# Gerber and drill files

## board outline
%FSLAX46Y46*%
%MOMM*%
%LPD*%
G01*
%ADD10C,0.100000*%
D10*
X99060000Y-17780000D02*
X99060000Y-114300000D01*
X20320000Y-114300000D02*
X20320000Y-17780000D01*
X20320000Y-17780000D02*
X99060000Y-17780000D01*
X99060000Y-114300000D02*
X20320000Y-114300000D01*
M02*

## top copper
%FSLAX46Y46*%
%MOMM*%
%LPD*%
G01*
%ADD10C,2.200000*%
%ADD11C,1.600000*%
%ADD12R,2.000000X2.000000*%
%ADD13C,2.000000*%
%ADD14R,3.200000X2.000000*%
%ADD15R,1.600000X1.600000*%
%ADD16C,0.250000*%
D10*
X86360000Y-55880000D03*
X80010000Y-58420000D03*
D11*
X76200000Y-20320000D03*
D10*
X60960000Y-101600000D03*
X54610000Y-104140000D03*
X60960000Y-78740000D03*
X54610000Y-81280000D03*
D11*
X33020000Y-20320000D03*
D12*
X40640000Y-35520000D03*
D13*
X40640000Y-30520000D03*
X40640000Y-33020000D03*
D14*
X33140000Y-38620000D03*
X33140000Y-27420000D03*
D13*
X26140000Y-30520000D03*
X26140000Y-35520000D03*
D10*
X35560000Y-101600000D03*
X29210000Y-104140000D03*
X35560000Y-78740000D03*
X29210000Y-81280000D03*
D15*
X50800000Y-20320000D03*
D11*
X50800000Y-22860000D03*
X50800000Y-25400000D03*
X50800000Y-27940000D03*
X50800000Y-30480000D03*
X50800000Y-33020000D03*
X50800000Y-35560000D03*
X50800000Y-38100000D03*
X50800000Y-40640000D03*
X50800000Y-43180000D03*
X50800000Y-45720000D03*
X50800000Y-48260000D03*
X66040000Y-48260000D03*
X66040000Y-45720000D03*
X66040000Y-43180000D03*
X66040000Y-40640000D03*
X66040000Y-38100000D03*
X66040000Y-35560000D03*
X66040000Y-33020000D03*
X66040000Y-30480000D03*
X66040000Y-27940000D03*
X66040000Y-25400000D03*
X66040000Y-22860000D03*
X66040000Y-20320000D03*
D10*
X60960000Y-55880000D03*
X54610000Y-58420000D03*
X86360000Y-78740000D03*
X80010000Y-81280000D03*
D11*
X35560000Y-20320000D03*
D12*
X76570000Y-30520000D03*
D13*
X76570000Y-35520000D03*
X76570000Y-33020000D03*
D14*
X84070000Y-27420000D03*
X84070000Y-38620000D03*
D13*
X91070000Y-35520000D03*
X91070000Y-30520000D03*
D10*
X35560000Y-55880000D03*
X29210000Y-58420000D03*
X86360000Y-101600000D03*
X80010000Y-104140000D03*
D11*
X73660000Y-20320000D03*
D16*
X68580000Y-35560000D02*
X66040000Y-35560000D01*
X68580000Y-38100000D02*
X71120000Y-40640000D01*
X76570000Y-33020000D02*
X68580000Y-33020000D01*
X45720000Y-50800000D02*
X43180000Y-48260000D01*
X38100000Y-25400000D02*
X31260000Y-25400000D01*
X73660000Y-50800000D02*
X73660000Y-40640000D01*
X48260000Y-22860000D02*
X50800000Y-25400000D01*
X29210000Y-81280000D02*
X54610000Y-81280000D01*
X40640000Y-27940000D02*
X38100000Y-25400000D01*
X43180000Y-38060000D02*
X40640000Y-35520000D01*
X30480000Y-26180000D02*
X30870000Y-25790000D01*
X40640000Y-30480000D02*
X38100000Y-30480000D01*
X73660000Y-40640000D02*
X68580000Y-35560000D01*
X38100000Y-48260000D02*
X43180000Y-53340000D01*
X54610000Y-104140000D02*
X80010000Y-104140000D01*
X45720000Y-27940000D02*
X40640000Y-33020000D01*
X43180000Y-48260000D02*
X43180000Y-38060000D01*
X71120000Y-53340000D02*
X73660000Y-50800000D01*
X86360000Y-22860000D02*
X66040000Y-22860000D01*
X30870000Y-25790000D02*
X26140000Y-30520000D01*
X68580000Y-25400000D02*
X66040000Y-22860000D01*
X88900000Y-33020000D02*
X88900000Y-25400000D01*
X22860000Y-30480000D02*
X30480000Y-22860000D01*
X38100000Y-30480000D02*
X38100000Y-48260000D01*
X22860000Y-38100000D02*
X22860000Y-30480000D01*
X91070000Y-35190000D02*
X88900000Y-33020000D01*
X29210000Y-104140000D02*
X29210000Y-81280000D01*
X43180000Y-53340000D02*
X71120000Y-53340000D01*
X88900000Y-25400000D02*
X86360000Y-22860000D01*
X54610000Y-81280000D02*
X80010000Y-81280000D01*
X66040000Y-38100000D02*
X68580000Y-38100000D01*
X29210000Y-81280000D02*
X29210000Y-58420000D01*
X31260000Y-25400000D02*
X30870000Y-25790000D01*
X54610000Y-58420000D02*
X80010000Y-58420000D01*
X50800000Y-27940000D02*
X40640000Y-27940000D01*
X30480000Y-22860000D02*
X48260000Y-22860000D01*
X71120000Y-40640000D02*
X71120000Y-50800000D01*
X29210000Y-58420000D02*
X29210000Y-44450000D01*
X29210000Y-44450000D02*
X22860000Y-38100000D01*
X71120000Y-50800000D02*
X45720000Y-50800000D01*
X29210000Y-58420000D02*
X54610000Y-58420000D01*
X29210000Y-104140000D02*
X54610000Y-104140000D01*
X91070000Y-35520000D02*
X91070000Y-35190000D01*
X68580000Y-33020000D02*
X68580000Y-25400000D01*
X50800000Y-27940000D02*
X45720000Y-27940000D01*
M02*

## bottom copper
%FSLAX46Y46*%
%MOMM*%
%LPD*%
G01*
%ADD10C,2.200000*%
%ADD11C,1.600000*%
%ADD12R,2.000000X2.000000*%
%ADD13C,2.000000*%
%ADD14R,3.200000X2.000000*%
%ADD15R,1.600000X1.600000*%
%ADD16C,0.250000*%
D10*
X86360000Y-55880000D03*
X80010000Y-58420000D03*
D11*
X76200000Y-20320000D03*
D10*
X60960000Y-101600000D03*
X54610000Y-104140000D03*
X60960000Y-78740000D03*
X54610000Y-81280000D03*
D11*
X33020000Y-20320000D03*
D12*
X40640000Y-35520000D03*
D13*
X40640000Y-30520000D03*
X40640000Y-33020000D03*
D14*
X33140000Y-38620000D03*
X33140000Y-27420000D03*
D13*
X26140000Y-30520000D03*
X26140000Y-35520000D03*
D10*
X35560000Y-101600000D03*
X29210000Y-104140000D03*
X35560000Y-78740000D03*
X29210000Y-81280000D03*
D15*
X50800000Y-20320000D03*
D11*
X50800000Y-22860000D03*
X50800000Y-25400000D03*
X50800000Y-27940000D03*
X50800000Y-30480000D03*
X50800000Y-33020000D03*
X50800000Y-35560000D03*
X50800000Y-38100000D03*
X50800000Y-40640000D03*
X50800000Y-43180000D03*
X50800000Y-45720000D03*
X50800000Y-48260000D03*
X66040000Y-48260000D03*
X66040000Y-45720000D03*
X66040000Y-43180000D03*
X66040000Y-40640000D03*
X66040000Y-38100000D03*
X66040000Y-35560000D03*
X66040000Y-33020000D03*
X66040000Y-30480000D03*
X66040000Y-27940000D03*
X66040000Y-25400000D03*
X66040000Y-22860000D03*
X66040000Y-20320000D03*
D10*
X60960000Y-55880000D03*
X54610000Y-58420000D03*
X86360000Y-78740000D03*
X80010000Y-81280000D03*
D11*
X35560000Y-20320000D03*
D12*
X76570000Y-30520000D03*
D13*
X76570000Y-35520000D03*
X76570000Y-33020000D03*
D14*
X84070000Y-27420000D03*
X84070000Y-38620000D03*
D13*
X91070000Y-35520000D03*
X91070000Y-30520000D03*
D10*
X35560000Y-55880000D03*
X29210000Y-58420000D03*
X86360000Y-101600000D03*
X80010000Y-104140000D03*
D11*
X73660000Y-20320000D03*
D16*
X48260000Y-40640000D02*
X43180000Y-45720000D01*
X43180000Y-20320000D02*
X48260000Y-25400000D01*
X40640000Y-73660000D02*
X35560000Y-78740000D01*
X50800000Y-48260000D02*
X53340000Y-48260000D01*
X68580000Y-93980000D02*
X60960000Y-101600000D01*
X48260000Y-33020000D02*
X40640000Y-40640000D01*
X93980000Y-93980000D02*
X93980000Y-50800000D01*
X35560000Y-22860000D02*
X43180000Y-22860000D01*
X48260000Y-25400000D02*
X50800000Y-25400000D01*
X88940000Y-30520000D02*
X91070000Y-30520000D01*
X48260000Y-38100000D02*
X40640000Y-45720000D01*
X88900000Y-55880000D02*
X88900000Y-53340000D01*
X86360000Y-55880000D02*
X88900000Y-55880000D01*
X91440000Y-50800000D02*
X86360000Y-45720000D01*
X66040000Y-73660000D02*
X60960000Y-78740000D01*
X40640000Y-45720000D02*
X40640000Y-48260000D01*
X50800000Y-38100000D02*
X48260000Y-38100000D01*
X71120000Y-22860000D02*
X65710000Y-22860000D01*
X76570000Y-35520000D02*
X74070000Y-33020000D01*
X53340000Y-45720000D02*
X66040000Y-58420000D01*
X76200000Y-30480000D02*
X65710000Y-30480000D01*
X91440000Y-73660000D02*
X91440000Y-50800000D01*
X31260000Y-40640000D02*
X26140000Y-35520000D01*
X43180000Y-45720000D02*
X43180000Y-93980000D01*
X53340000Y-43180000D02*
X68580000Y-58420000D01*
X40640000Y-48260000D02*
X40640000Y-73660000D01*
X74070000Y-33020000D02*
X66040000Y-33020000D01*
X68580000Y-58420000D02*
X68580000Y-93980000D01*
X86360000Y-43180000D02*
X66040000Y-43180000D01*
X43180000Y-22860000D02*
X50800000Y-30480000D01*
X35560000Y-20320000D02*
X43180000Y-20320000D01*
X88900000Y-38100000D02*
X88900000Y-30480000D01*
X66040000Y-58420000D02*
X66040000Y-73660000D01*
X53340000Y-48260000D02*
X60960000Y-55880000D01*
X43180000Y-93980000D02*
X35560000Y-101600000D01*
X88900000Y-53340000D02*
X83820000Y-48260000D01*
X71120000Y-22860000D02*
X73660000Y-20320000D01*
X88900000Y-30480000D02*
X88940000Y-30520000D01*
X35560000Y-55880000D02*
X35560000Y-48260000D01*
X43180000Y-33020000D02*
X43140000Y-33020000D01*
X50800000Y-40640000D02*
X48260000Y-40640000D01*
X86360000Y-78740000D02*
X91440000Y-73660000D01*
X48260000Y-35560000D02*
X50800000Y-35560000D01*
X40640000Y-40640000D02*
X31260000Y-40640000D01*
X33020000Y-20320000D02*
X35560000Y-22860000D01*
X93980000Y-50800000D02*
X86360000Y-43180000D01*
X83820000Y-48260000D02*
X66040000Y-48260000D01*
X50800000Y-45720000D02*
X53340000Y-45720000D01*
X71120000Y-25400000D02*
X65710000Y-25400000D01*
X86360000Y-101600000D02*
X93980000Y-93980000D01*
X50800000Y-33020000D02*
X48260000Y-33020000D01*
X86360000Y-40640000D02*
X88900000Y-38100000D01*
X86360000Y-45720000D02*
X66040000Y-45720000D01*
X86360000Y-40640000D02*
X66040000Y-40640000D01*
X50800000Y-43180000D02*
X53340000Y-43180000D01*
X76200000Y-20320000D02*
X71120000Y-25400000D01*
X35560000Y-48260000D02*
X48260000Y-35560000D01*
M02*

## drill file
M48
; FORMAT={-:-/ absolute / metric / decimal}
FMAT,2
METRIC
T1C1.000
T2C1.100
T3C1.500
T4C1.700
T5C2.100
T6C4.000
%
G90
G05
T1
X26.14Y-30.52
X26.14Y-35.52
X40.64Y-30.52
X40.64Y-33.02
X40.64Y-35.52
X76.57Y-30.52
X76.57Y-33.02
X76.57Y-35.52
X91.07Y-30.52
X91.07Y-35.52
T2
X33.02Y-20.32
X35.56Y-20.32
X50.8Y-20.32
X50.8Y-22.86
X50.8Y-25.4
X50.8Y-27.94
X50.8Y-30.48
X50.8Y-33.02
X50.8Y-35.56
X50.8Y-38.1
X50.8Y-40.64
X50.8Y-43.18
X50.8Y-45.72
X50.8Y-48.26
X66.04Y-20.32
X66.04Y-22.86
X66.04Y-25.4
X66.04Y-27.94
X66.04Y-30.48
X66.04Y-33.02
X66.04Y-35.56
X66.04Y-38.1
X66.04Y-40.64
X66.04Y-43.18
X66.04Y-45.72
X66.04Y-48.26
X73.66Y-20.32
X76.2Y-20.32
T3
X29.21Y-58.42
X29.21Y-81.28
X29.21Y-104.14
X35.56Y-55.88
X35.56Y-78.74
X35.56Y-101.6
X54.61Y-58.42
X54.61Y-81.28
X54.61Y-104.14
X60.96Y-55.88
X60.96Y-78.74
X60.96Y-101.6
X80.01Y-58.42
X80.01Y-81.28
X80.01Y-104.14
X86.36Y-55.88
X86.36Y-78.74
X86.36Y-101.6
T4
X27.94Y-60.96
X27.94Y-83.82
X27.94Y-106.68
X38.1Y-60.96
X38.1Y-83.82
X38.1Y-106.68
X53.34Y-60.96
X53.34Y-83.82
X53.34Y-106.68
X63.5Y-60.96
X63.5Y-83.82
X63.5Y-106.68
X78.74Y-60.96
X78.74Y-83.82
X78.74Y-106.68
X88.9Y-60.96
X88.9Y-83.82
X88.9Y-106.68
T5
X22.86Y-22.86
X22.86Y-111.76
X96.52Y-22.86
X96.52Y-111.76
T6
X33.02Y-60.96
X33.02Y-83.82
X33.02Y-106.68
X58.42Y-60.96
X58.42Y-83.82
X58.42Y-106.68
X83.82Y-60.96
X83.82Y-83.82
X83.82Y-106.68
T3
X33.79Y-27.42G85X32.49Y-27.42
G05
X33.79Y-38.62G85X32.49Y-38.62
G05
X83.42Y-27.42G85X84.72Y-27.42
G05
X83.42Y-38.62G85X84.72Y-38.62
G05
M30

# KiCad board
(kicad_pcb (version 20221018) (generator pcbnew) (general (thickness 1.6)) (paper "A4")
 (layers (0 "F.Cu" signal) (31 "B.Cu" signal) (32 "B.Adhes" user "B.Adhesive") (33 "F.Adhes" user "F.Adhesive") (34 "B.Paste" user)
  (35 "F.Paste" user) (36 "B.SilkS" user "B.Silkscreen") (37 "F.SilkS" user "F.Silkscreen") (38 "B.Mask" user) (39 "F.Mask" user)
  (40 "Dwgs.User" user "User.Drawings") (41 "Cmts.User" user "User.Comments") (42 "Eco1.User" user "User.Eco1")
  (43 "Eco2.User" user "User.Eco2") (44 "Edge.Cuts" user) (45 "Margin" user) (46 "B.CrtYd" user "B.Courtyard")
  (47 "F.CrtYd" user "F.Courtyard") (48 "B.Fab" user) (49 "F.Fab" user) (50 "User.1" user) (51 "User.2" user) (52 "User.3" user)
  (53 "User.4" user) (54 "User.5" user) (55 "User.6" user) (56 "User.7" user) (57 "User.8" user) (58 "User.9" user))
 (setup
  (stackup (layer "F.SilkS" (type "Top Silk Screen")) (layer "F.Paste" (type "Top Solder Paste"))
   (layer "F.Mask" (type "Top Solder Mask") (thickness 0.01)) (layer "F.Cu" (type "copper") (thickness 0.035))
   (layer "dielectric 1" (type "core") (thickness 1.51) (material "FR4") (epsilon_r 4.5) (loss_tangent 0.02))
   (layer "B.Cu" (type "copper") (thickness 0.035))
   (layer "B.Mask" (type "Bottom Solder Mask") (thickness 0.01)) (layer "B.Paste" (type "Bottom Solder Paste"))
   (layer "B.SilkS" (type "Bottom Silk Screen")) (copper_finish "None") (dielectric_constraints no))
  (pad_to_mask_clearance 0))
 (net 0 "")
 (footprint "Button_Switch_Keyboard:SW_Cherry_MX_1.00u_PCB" (layer "F.Cu") (at 86.36 55.88)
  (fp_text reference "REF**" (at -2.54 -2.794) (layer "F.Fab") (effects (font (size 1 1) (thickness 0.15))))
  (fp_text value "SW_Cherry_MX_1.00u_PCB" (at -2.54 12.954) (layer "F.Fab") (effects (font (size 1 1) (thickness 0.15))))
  (pad "" np_thru_hole circle (at -7.62 5.08) (size 1.7 1.7) (drill 1.7) (layers "F&B.Cu" "*.Mask"))
  (pad "" np_thru_hole circle (at -2.54 5.08) (size 4 4) (drill 4) (layers "F&B.Cu" "*.Mask"))
  (pad "" np_thru_hole circle (at 2.54 5.08) (size 1.7 1.7) (drill 1.7) (layers "F&B.Cu" "*.Mask"))
  (pad "1" thru_hole circle (at 0 0) (size 2.2 2.2) (drill 1.5) (layers "*.Cu" "*.Mask"))
  (pad "2" thru_hole circle (at -6.35 2.54) (size 2.2 2.2) (drill 1.5) (layers "*.Cu" "*.Mask")))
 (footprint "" (layer "F.Cu") (at 76.2 20.32)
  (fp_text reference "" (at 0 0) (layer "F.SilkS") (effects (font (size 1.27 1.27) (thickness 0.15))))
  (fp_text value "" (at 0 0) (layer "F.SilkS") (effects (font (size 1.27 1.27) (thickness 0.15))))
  (pad "24" thru_hole circle (at 0 0 270) (size 1.6 1.6) (drill 1.1) (layers "*.Cu" "*.Mask" "F.SilkS")))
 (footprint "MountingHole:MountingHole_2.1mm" (layer "F.Cu") (at 96.52 22.86)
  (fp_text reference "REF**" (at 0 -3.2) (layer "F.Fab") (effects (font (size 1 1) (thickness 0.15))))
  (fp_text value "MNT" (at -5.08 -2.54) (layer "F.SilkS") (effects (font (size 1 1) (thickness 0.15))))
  (pad "" np_thru_hole circle (at 0 0) (size 2.1 2.1) (drill 2.1) (layers "F&B.Cu" "*.Mask")))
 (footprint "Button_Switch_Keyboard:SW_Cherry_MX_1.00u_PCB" (layer "F.Cu") (at 60.96 101.6)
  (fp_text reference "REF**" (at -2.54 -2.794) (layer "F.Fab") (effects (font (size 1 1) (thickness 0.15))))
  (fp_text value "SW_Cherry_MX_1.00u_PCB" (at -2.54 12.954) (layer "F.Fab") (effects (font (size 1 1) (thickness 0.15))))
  (pad "" np_thru_hole circle (at -7.62 5.08) (size 1.7 1.7) (drill 1.7) (layers "F&B.Cu" "*.Mask"))
  (pad "" np_thru_hole circle (at -2.54 5.08) (size 4 4) (drill 4) (layers "F&B.Cu" "*.Mask"))
  (pad "" np_thru_hole circle (at 2.54 5.08) (size 1.7 1.7) (drill 1.7) (layers "F&B.Cu" "*.Mask"))
  (pad "1" thru_hole circle (at 0 0) (size 2.2 2.2) (drill 1.5) (layers "*.Cu" "*.Mask"))
  (pad "2" thru_hole circle (at -6.35 2.54) (size 2.2 2.2) (drill 1.5) (layers "*.Cu" "*.Mask")))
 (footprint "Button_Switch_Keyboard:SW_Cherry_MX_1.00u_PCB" (layer "F.Cu") (at 60.96 78.74)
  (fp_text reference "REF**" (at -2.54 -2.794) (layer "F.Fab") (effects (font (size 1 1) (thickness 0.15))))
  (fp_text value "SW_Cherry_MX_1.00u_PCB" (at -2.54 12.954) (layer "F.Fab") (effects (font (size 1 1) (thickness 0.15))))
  (pad "" np_thru_hole circle (at -7.62 5.08) (size 1.7 1.7) (drill 1.7) (layers "F&B.Cu" "*.Mask"))
  (pad "" np_thru_hole circle (at -2.54 5.08) (size 4 4) (drill 4) (layers "F&B.Cu" "*.Mask"))
  (pad "" np_thru_hole circle (at 2.54 5.08) (size 1.7 1.7) (drill 1.7) (layers "F&B.Cu" "*.Mask"))
  (pad "1" thru_hole circle (at 0 0) (size 2.2 2.2) (drill 1.5) (layers "*.Cu" "*.Mask"))
  (pad "2" thru_hole circle (at -6.35 2.54) (size 2.2 2.2) (drill 1.5) (layers "*.Cu" "*.Mask")))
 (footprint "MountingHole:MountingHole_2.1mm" (layer "F.Cu") (at 96.52 111.76)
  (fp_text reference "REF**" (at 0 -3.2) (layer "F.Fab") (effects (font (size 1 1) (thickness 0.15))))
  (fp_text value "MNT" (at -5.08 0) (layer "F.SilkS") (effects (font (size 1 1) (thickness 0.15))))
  (pad "" np_thru_hole circle (at 0 0) (size 2.1 2.1) (drill 2.1) (layers "F&B.Cu" "*.Mask")))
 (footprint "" (layer "F.Cu") (at 33.02 20.32)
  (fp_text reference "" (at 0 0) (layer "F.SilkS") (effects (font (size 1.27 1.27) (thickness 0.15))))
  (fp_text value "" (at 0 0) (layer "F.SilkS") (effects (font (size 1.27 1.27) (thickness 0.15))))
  (pad "24" thru_hole circle (at 0 0 270) (size 1.6 1.6) (drill 1.1) (layers "*.Cu" "*.Mask" "F.SilkS")))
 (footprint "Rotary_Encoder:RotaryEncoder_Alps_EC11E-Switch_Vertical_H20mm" (layer "F.Cu") (at 40.64 35.52 180)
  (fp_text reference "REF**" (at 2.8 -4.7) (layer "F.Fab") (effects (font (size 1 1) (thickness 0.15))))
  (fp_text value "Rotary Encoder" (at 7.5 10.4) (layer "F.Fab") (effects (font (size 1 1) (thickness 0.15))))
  (pad "A" thru_hole rect (at 0 0 180) (size 2 2) (drill 1) (layers "*.Cu" "*.Mask"))
  (pad "B" thru_hole circle (at 0 5 180) (size 2 2) (drill 1) (layers "*.Cu" "*.Mask"))
  (pad "C" thru_hole circle (at 0 2.5 180) (size 2 2) (drill 1) (layers "*.Cu" "*.Mask"))
  (pad "MP" thru_hole rect (at 7.5 -3.1 180) (size 3.2 2) (drill oval 2.8 1.5) (layers "*.Cu" "*.Mask"))
  (pad "MP" thru_hole rect (at 7.5 8.1 180) (size 3.2 2) (drill oval 2.8 1.5) (layers "*.Cu" "*.Mask"))
  (pad "S1" thru_hole circle (at 14.5 5 180) (size 2 2) (drill 1) (layers "*.Cu" "*.Mask"))
  (pad "S2" thru_hole circle (at 14.5 0 180) (size 2 2) (drill 1) (layers "*.Cu" "*.Mask")))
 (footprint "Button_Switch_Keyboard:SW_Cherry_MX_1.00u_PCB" (layer "F.Cu") (at 35.56 101.6)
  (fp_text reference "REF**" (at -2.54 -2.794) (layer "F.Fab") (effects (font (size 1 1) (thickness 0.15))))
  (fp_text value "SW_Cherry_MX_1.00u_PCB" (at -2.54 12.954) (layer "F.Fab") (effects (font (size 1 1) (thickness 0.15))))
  (pad "" np_thru_hole circle (at -7.62 5.08) (size 1.7 1.7) (drill 1.7) (layers "F&B.Cu" "*.Mask"))
  (pad "" np_thru_hole circle (at -2.54 5.08) (size 4 4) (drill 4) (layers "F&B.Cu" "*.Mask"))
  (pad "" np_thru_hole circle (at 2.54 5.08) (size 1.7 1.7) (drill 1.7) (layers "F&B.Cu" "*.Mask"))
  (pad "1" thru_hole circle (at 0 0) (size 2.2 2.2) (drill 1.5) (layers "*.Cu" "*.Mask"))
  (pad "2" thru_hole circle (at -6.35 2.54) (size 2.2 2.2) (drill 1.5) (layers "*.Cu" "*.Mask")))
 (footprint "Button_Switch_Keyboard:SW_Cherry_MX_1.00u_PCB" (layer "F.Cu") (at 35.56 78.74)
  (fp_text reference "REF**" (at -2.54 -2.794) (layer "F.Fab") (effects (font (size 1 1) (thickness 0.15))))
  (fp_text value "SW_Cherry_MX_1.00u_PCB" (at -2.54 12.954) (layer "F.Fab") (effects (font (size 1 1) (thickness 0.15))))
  (pad "" np_thru_hole circle (at -7.62 5.08) (size 1.7 1.7) (drill 1.7) (layers "F&B.Cu" "*.Mask"))
  (pad "" np_thru_hole circle (at -2.54 5.08) (size 4 4) (drill 4) (layers "F&B.Cu" "*.Mask"))
  (pad "" np_thru_hole circle (at 2.54 5.08) (size 1.7 1.7) (drill 1.7) (layers "F&B.Cu" "*.Mask"))
  (pad "1" thru_hole circle (at 0 0) (size 2.2 2.2) (drill 1.5) (layers "*.Cu" "*.Mask"))
  (pad "2" thru_hole circle (at -6.35 2.54) (size 2.2 2.2) (drill 1.5) (layers "*.Cu" "*.Mask")))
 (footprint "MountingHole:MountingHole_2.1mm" (layer "F.Cu") (at 22.86 111.76)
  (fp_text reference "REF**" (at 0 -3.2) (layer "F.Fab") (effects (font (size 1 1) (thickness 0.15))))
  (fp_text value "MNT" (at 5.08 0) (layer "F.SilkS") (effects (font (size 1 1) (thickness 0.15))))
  (pad "" np_thru_hole circle (at 0 0) (size 2.1 2.1) (drill 2.1) (layers "F&B.Cu" "*.Mask")))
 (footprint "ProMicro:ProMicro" (layer "F.Cu") (at 58.42 34.29 -90)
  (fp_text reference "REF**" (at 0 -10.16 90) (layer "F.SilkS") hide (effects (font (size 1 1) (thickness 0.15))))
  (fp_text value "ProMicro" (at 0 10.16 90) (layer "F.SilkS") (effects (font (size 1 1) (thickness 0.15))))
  (pad "1" thru_hole rect (at -13.97 7.62 270) (size 1.6 1.6) (drill 1.1) (layers "*.Cu" "*.Mask" "F.SilkS"))
  (pad "2" thru_hole circle (at -11.43 7.62 270) (size 1.6 1.6) (drill 1.1) (layers "*.Cu" "*.Mask" "F.SilkS"))
  (pad "3" thru_hole circle (at -8.89 7.62 270) (size 1.6 1.6) (drill 1.1) (layers "*.Cu" "*.Mask" "F.SilkS"))
  (pad "4" thru_hole circle (at -6.35 7.62 270) (size 1.6 1.6) (drill 1.1) (layers "*.Cu" "*.Mask" "F.SilkS"))
  (pad "5" thru_hole circle (at -3.81 7.62 270) (size 1.6 1.6) (drill 1.1) (layers "*.Cu" "*.Mask" "F.SilkS"))
  (pad "6" thru_hole circle (at -1.27 7.62 270) (size 1.6 1.6) (drill 1.1) (layers "*.Cu" "*.Mask" "F.SilkS"))
  (pad "7" thru_hole circle (at 1.27 7.62 270) (size 1.6 1.6) (drill 1.1) (layers "*.Cu" "*.Mask" "F.SilkS"))
  (pad "8" thru_hole circle (at 3.81 7.62 270) (size 1.6 1.6) (drill 1.1) (layers "*.Cu" "*.Mask" "F.SilkS"))
  (pad "9" thru_hole circle (at 6.35 7.62 270) (size 1.6 1.6) (drill 1.1) (layers "*.Cu" "*.Mask" "F.SilkS"))
  (pad "10" thru_hole circle (at 8.89 7.62 270) (size 1.6 1.6) (drill 1.1) (layers "*.Cu" "*.Mask" "F.SilkS"))
  (pad "11" thru_hole circle (at 11.43 7.62 270) (size 1.6 1.6) (drill 1.1) (layers "*.Cu" "*.Mask" "F.SilkS"))
  (pad "12" thru_hole circle (at 13.97 7.62 270) (size 1.6 1.6) (drill 1.1) (layers "*.Cu" "*.Mask" "F.SilkS"))
  (pad "13" thru_hole circle (at 13.97 -7.62 270) (size 1.6 1.6) (drill 1.1) (layers "*.Cu" "*.Mask" "F.SilkS"))
  (pad "14" thru_hole circle (at 11.43 -7.62 270) (size 1.6 1.6) (drill 1.1) (layers "*.Cu" "*.Mask" "F.SilkS"))
  (pad "15" thru_hole circle (at 8.89 -7.62 270) (size 1.6 1.6) (drill 1.1) (layers "*.Cu" "*.Mask" "F.SilkS"))
  (pad "16" thru_hole circle (at 6.35 -7.62 270) (size 1.6 1.6) (drill 1.1) (layers "*.Cu" "*.Mask" "F.SilkS"))
  (pad "17" thru_hole circle (at 3.81 -7.62 270) (size 1.6 1.6) (drill 1.1) (layers "*.Cu" "*.Mask" "F.SilkS"))
  (pad "18" thru_hole circle (at 1.27 -7.62 270) (size 1.6 1.6) (drill 1.1) (layers "*.Cu" "*.Mask" "F.SilkS"))
  (pad "19" thru_hole circle (at -1.27 -7.62 270) (size 1.6 1.6) (drill 1.1) (layers "*.Cu" "*.Mask" "F.SilkS"))
  (pad "20" thru_hole circle (at -3.81 -7.62 270) (size 1.6 1.6) (drill 1.1) (layers "*.Cu" "*.Mask" "F.SilkS"))
  (pad "21" thru_hole circle (at -6.35 -7.62 270) (size 1.6 1.6) (drill 1.1) (layers "*.Cu" "*.Mask" "F.SilkS"))
  (pad "22" thru_hole circle (at -8.89 -7.62 270) (size 1.6 1.6) (drill 1.1) (layers "*.Cu" "*.Mask" "F.SilkS"))
  (pad "23" thru_hole circle (at -11.43 -7.62 270) (size 1.6 1.6) (drill 1.1) (layers "*.Cu" "*.Mask" "F.SilkS"))
  (pad "24" thru_hole circle (at -13.97 -7.62 270) (size 1.6 1.6) (drill 1.1) (layers "*.Cu" "*.Mask" "F.SilkS")))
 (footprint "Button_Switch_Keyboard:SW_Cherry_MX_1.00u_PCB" (layer "F.Cu") (at 60.96 55.88)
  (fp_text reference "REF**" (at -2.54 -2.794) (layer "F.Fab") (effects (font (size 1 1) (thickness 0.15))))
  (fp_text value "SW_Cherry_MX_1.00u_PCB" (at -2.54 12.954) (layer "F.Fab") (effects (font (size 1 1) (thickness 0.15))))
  (pad "" np_thru_hole circle (at -7.62 5.08) (size 1.7 1.7) (drill 1.7) (layers "F&B.Cu" "*.Mask"))
  (pad "" np_thru_hole circle (at -2.54 5.08) (size 4 4) (drill 4) (layers "F&B.Cu" "*.Mask"))
  (pad "" np_thru_hole circle (at 2.54 5.08) (size 1.7 1.7) (drill 1.7) (layers "F&B.Cu" "*.Mask"))
  (pad "1" thru_hole circle (at 0 0) (size 2.2 2.2) (drill 1.5) (layers "*.Cu" "*.Mask"))
  (pad "2" thru_hole circle (at -6.35 2.54) (size 2.2 2.2) (drill 1.5) (layers "*.Cu" "*.Mask")))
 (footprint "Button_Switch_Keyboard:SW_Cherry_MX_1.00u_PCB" (layer "F.Cu") (at 86.36 78.74)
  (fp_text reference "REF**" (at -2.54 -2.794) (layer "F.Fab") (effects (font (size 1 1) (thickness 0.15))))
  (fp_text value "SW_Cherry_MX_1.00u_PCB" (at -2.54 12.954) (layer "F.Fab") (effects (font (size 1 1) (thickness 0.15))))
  (pad "" np_thru_hole circle (at -7.62 5.08) (size 1.7 1.7) (drill 1.7) (layers "F&B.Cu" "*.Mask"))
  (pad "" np_thru_hole circle (at -2.54 5.08) (size 4 4) (drill 4) (layers "F&B.Cu" "*.Mask"))
  (pad "" np_thru_hole circle (at 2.54 5.08) (size 1.7 1.7) (drill 1.7) (layers "F&B.Cu" "*.Mask"))
  (pad "1" thru_hole circle (at 0 0) (size 2.2 2.2) (drill 1.5) (layers "*.Cu" "*.Mask"))
  (pad "2" thru_hole circle (at -6.35 2.54) (size 2.2 2.2) (drill 1.5) (layers "*.Cu" "*.Mask")))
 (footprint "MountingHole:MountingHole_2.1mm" (layer "F.Cu") (at 22.86 22.86)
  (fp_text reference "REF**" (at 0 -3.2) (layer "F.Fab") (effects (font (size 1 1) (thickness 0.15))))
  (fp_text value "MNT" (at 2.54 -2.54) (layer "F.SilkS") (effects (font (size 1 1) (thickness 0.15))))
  (pad "" np_thru_hole circle (at 0 0) (size 2.1 2.1) (drill 2.1) (layers "*.Cu" "*.Mask")))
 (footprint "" (layer "F.Cu") (at 35.56 20.32)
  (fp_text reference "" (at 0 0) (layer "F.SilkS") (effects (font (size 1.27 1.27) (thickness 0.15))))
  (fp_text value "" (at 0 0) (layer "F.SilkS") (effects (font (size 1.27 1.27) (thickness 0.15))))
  (pad "24" thru_hole circle (at 0 0 270) (size 1.6 1.6) (drill 1.1) (layers "*.Cu" "*.Mask" "F.SilkS")))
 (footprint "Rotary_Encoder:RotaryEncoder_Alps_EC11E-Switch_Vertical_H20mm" (layer "F.Cu") (at 76.57 30.52)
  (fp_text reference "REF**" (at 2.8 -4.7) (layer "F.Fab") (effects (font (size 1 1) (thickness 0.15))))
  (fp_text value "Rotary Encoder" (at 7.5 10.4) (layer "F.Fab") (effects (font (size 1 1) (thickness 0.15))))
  (pad "A" thru_hole rect (at 0 0) (size 2 2) (drill 1) (layers "*.Cu" "*.Mask"))
  (pad "B" thru_hole circle (at 0 5) (size 2 2) (drill 1) (layers "*.Cu" "*.Mask"))
  (pad "C" thru_hole circle (at 0 2.5) (size 2 2) (drill 1) (layers "*.Cu" "*.Mask"))
  (pad "MP" thru_hole rect (at 7.5 -3.1) (size 3.2 2) (drill oval 2.8 1.5) (layers "*.Cu" "*.Mask"))
  (pad "MP" thru_hole rect (at 7.5 8.1) (size 3.2 2) (drill oval 2.8 1.5) (layers "*.Cu" "*.Mask"))
  (pad "S1" thru_hole circle (at 14.5 5) (size 2 2) (drill 1) (layers "*.Cu" "*.Mask"))
  (pad "S2" thru_hole circle (at 14.5 0) (size 2 2) (drill 1) (layers "*.Cu" "*.Mask")))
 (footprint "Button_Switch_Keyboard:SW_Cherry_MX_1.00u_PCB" (layer "F.Cu") (at 35.56 55.88)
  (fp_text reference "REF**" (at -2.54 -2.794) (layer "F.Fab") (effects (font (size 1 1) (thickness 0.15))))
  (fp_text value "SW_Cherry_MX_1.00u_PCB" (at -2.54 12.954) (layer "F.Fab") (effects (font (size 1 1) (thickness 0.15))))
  (pad "" np_thru_hole circle (at -7.62 5.08) (size 1.7 1.7) (drill 1.7) (layers "F&B.Cu" "*.Mask"))
  (pad "" np_thru_hole circle (at -2.54 5.08) (size 4 4) (drill 4) (layers "F&B.Cu" "*.Mask"))
  (pad "" np_thru_hole circle (at 2.54 5.08) (size 1.7 1.7) (drill 1.7) (layers "F&B.Cu" "*.Mask"))
  (pad "1" thru_hole circle (at 0 0) (size 2.2 2.2) (drill 1.5) (layers "*.Cu" "*.Mask"))
  (pad "2" thru_hole circle (at -6.35 2.54) (size 2.2 2.2) (drill 1.5) (layers "*.Cu" "*.Mask")))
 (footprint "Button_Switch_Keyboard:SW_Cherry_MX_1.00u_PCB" (layer "F.Cu") (at 86.36 101.6)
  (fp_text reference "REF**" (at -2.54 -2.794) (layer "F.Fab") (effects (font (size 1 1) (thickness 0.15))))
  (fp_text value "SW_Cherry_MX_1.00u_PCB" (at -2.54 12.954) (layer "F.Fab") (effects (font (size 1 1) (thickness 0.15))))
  (pad "" np_thru_hole circle (at -7.62 5.08) (size 1.7 1.7) (drill 1.7) (layers "F&B.Cu" "*.Mask"))
  (pad "" np_thru_hole circle (at -2.54 5.08) (size 4 4) (drill 4) (layers "F&B.Cu" "*.Mask"))
  (pad "" np_thru_hole circle (at 2.54 5.08) (size 1.7 1.7) (drill 1.7) (layers "F&B.Cu" "*.Mask"))
  (pad "1" thru_hole circle (at 0 0) (size 2.2 2.2) (drill 1.5) (layers "*.Cu" "*.Mask"))
  (pad "2" thru_hole circle (at -6.35 2.54) (size 2.2 2.2) (drill 1.5) (layers "*.Cu" "*.Mask")))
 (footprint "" (layer "F.Cu") (at 73.66 20.32)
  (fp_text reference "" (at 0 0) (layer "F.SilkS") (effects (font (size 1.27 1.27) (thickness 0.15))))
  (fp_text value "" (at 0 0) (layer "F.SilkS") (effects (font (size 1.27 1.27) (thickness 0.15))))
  (pad "24" thru_hole circle (at 0 0 270) (size 1.6 1.6) (drill 1.1) (layers "*.Cu" "*.Mask" "F.SilkS")))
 (gr_line (start 99.06 17.78) (end 99.06 114.3) (stroke (width 0.1) (type default)) (layer "Edge.Cuts"))
 (gr_line (start 20.32 114.3) (end 20.32 17.78) (stroke (width 0.1) (type default)) (layer "Edge.Cuts"))
 (gr_line (start 20.32 17.78) (end 99.06 17.78) (stroke (width 0.1) (type default)) (layer "Edge.Cuts"))
 (gr_line (start 99.06 114.3) (end 20.32 114.3) (stroke (width 0.1) (type default)) (layer "Edge.Cuts"))
 (segment (start 68.58 35.56) (end 66.04 35.56) (width 0.25) (layer "F.Cu") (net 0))
 (segment (start 68.58 38.1) (end 71.12 40.64) (width 0.25) (layer "F.Cu") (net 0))
 (segment (start 76.57 33.02) (end 68.58 33.02) (width 0.25) (layer "F.Cu") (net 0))
 (segment (start 45.72 50.8) (end 43.18 48.26) (width 0.25) (layer "F.Cu") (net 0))
 (segment (start 38.1 25.4) (end 31.26 25.4) (width 0.25) (layer "F.Cu") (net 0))
 (segment (start 73.66 50.8) (end 73.66 40.64) (width 0.25) (layer "F.Cu") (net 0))
 (segment (start 48.26 22.86) (end 50.8 25.4) (width 0.25) (layer "F.Cu") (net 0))
 (segment (start 29.21 81.28) (end 54.61 81.28) (width 0.25) (layer "F.Cu") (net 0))
 (segment (start 40.64 27.94) (end 38.1 25.4) (width 0.25) (layer "F.Cu") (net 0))
 (segment (start 43.18 38.06) (end 40.64 35.52) (width 0.25) (layer "F.Cu") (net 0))
 (segment (start 30.48 26.18) (end 30.87 25.79) (width 0.25) (layer "F.Cu") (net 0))
 (segment (start 40.64 30.48) (end 38.1 30.48) (width 0.25) (layer "F.Cu") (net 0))
 (segment (start 73.66 40.64) (end 68.58 35.56) (width 0.25) (layer "F.Cu") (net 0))
 (segment (start 38.1 48.26) (end 43.18 53.34) (width 0.25) (layer "F.Cu") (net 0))
 (segment (start 54.61 104.14) (end 80.01 104.14) (width 0.25) (layer "F.Cu") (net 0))
 (segment (start 45.72 27.94) (end 40.64 33.02) (width 0.25) (layer "F.Cu") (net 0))
 (segment (start 43.18 48.26) (end 43.18 38.06) (width 0.25) (layer "F.Cu") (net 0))
 (segment (start 71.12 53.34) (end 73.66 50.8) (width 0.25) (layer "F.Cu") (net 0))
 (segment (start 86.36 22.86) (end 66.04 22.86) (width 0.25) (layer "F.Cu") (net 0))
 (segment (start 30.87 25.79) (end 26.14 30.52) (width 0.25) (layer "F.Cu") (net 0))
 (segment (start 68.58 25.4) (end 66.04 22.86) (width 0.25) (layer "F.Cu") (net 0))
 (segment (start 88.9 33.02) (end 88.9 25.4) (width 0.25) (layer "F.Cu") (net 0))
 (segment (start 22.86 30.48) (end 30.48 22.86) (width 0.25) (layer "F.Cu") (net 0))
 (segment (start 38.1 30.48) (end 38.1 48.26) (width 0.25) (layer "F.Cu") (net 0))
 (segment (start 22.86 38.1) (end 22.86 30.48) (width 0.25) (layer "F.Cu") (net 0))
 (segment (start 91.07 35.19) (end 88.9 33.02) (width 0.25) (layer "F.Cu") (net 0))
 (segment (start 29.21 104.14) (end 29.21 81.28) (width 0.25) (layer "F.Cu") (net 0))
 (segment (start 43.18 53.34) (end 71.12 53.34) (width 0.25) (layer "F.Cu") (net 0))
 (segment (start 88.9 25.4) (end 86.36 22.86) (width 0.25) (layer "F.Cu") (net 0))
 (segment (start 54.61 81.28) (end 80.01 81.28) (width 0.25) (layer "F.Cu") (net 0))
 (segment (start 66.04 38.1) (end 68.58 38.1) (width 0.25) (layer "F.Cu") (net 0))
 (segment (start 29.21 81.28) (end 29.21 58.42) (width 0.25) (layer "F.Cu") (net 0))
 (segment (start 31.26 25.4) (end 30.87 25.79) (width 0.25) (layer "F.Cu") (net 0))
 (segment (start 54.61 58.42) (end 80.01 58.42) (width 0.25) (layer "F.Cu") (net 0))
 (segment (start 50.8 27.94) (end 40.64 27.94) (width 0.25) (layer "F.Cu") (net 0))
 (segment (start 30.48 22.86) (end 48.26 22.86) (width 0.25) (layer "F.Cu") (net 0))
 (segment (start 71.12 40.64) (end 71.12 50.8) (width 0.25) (layer "F.Cu") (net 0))
 (segment (start 29.21 58.42) (end 29.21 44.45) (width 0.25) (layer "F.Cu") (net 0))
 (segment (start 29.21 44.45) (end 22.86 38.1) (width 0.25) (layer "F.Cu") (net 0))
 (segment (start 71.12 50.8) (end 45.72 50.8) (width 0.25) (layer "F.Cu") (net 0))
 (segment (start 29.21 58.42) (end 54.61 58.42) (width 0.25) (layer "F.Cu") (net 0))
 (segment (start 29.21 104.14) (end 54.61 104.14) (width 0.25) (layer "F.Cu") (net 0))
 (segment (start 91.07 35.52) (end 91.07 35.19) (width 0.25) (layer "F.Cu") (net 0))
 (segment (start 68.58 33.02) (end 68.58 25.4) (width 0.25) (layer "F.Cu") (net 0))
 (segment (start 50.8 27.94) (end 45.72 27.94) (width 0.25) (layer "F.Cu") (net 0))
 (segment (start 48.26 40.64) (end 43.18 45.72) (width 0.25) (layer "B.Cu") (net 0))
 (segment (start 43.18 20.32) (end 48.26 25.4) (width 0.25) (layer "B.Cu") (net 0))
 (segment (start 40.64 73.66) (end 35.56 78.74) (width 0.25) (layer "B.Cu") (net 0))
 (segment (start 50.8 48.26) (end 53.34 48.26) (width 0.25) (layer "B.Cu") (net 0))
 (segment (start 68.58 93.98) (end 60.96 101.6) (width 0.25) (layer "B.Cu") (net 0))
 (segment (start 48.26 33.02) (end 40.64 40.64) (width 0.25) (layer "B.Cu") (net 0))
 (segment (start 93.98 93.98) (end 93.98 50.8) (width 0.25) (layer "B.Cu") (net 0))
 (segment (start 35.56 22.86) (end 43.18 22.86) (width 0.25) (layer "B.Cu") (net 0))
 (segment (start 48.26 25.4) (end 50.8 25.4) (width 0.25) (layer "B.Cu") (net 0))
 (segment (start 88.94 30.52) (end 91.07 30.52) (width 0.25) (layer "B.Cu") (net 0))
 (segment (start 48.26 38.1) (end 40.64 45.72) (width 0.25) (layer "B.Cu") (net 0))
 (segment (start 88.9 55.88) (end 88.9 53.34) (width 0.25) (layer "B.Cu") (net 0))
 (segment (start 86.36 55.88) (end 88.9 55.88) (width 0.25) (layer "B.Cu") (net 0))
 (segment (start 91.44 50.8) (end 86.36 45.72) (width 0.25) (layer "B.Cu") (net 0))
 (segment (start 66.04 73.66) (end 60.96 78.74) (width 0.25) (layer "B.Cu") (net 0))
 (segment (start 40.64 45.72) (end 40.64 48.26) (width 0.25) (layer "B.Cu") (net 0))
 (segment (start 50.8 38.1) (end 48.26 38.1) (width 0.25) (layer "B.Cu") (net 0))
 (segment (start 71.12 22.86) (end 65.71 22.86) (width 0.25) (layer "B.Cu") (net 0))
 (segment (start 76.57 35.52) (end 74.07 33.02) (width 0.25) (layer "B.Cu") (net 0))
 (segment (start 53.34 45.72) (end 66.04 58.42) (width 0.25) (layer "B.Cu") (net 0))
 (segment (start 76.2 30.48) (end 65.71 30.48) (width 0.25) (layer "B.Cu") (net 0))
 (segment (start 91.44 73.66) (end 91.44 50.8) (width 0.25) (layer "B.Cu") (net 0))
 (segment (start 31.26 40.64) (end 26.14 35.52) (width 0.25) (layer "B.Cu") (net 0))
 (segment (start 43.18 45.72) (end 43.18 93.98) (width 0.25) (layer "B.Cu") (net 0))
 (segment (start 53.34 43.18) (end 68.58 58.42) (width 0.25) (layer "B.Cu") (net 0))
 (segment (start 40.64 48.26) (end 40.64 73.66) (width 0.25) (layer "B.Cu") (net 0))
 (segment (start 74.07 33.02) (end 66.04 33.02) (width 0.25) (layer "B.Cu") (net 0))
 (segment (start 68.58 58.42) (end 68.58 93.98) (width 0.25) (layer "B.Cu") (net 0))
 (segment (start 86.36 43.18) (end 66.04 43.18) (width 0.25) (layer "B.Cu") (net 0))
 (segment (start 43.18 22.86) (end 50.8 30.48) (width 0.25) (layer "B.Cu") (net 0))
 (segment (start 35.56 20.32) (end 43.18 20.32) (width 0.25) (layer "B.Cu") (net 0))
 (segment (start 88.9 38.1) (end 88.9 30.48) (width 0.25) (layer "B.Cu") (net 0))
 (segment (start 66.04 58.42) (end 66.04 73.66) (width 0.25) (layer "B.Cu") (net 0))
 (segment (start 53.34 48.26) (end 60.96 55.88) (width 0.25) (layer "B.Cu") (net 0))
 (segment (start 43.18 93.98) (end 35.56 101.6) (width 0.25) (layer "B.Cu") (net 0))
 (segment (start 88.9 53.34) (end 83.82 48.26) (width 0.25) (layer "B.Cu") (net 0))
 (segment (start 71.12 22.86) (end 73.66 20.32) (width 0.25) (layer "B.Cu") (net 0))
 (segment (start 88.9 30.48) (end 88.94 30.52) (width 0.25) (layer "B.Cu") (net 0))
 (segment (start 35.56 55.88) (end 35.56 48.26) (width 0.25) (layer "B.Cu") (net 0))
 (segment (start 43.18 33.02) (end 43.14 33.02) (width 0.25) (layer "B.Cu") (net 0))
 (segment (start 50.8 40.64) (end 48.26 40.64) (width 0.25) (layer "B.Cu") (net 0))
 (segment (start 86.36 78.74) (end 91.44 73.66) (width 0.25) (layer "B.Cu") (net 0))
 (segment (start 48.26 35.56) (end 50.8 35.56) (width 0.25) (layer "B.Cu") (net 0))
 (segment (start 40.64 40.64) (end 31.26 40.64) (width 0.25) (layer "B.Cu") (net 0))
 (segment (start 33.02 20.32) (end 35.56 22.86) (width 0.25) (layer "B.Cu") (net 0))
 (segment (start 93.98 50.8) (end 86.36 43.18) (width 0.25) (layer "B.Cu") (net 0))
 (segment (start 83.82 48.26) (end 66.04 48.26) (width 0.25) (layer "B.Cu") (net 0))
 (segment (start 50.8 45.72) (end 53.34 45.72) (width 0.25) (layer "B.Cu") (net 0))
 (segment (start 71.12 25.4) (end 65.71 25.4) (width 0.25) (layer "B.Cu") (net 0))
 (segment (start 86.36 101.6) (end 93.98 93.98) (width 0.25) (layer "B.Cu") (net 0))
 (segment (start 50.8 33.02) (end 48.26 33.02) (width 0.25) (layer "B.Cu") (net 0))
 (segment (start 86.36 40.64) (end 88.9 38.1) (width 0.25) (layer "B.Cu") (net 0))
 (segment (start 86.36 45.72) (end 66.04 45.72) (width 0.25) (layer "B.Cu") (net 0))
 (segment (start 86.36 40.64) (end 66.04 40.64) (width 0.25) (layer "B.Cu") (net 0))
 (segment (start 50.8 43.18) (end 53.34 43.18) (width 0.25) (layer "B.Cu") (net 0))
 (segment (start 76.2 20.32) (end 71.12 25.4) (width 0.25) (layer "B.Cu") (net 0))
 (segment (start 35.56 48.26) (end 48.26 35.56) (width 0.25) (layer "B.Cu") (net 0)))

